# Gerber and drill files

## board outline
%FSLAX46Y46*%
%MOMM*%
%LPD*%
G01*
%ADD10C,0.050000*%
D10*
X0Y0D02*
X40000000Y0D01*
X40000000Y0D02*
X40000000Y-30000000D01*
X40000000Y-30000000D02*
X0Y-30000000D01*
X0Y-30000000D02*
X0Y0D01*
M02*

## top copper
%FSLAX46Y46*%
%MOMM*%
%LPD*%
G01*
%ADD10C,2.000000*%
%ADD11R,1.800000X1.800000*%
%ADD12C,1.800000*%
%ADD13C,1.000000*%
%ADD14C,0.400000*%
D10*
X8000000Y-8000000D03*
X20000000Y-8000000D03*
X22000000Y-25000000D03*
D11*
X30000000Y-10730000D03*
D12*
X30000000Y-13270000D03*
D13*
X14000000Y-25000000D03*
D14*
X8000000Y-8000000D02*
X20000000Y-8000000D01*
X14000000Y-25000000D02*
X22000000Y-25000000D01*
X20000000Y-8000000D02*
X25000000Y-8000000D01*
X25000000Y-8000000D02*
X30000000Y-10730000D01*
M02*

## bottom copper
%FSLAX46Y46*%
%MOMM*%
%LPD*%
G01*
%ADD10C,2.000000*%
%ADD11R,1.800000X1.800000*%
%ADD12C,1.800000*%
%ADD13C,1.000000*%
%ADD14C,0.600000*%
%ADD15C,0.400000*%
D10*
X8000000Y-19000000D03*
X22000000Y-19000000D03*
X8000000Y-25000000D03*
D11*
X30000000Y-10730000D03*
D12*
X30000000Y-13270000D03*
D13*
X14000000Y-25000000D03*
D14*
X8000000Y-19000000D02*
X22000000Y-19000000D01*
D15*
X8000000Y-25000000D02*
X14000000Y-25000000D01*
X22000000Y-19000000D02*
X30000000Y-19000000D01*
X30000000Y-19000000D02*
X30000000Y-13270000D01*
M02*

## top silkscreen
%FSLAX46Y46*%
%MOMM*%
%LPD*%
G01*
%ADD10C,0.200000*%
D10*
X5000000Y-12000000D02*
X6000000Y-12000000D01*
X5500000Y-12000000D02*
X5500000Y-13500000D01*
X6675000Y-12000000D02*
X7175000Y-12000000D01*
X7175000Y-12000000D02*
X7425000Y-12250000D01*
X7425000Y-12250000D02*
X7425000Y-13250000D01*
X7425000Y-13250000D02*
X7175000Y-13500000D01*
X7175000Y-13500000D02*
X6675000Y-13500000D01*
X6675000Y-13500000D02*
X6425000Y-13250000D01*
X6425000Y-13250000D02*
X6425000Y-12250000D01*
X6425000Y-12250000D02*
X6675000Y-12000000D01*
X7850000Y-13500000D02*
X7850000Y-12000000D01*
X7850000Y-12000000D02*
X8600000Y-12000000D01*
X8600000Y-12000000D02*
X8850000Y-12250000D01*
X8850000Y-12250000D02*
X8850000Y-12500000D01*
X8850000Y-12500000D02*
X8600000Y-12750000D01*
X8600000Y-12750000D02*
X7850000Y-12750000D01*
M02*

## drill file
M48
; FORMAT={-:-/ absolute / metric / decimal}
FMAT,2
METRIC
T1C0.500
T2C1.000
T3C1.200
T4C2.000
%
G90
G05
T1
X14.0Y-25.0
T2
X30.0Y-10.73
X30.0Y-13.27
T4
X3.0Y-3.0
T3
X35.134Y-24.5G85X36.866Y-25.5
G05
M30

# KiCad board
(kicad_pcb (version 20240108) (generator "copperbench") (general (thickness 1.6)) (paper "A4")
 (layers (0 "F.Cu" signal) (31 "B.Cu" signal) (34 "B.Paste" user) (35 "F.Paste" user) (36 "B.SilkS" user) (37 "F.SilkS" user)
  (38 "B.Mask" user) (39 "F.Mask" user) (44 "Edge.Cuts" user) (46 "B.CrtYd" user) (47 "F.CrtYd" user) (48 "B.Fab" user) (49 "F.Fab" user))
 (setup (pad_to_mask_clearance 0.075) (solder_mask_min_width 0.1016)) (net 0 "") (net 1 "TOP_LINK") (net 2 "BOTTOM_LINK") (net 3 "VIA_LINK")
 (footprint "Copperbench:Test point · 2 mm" (layer "F.Cu") (at 8 8 0)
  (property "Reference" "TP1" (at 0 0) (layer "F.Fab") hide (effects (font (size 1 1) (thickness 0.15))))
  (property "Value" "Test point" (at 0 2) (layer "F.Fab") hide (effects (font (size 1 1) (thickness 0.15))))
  (pad "1" smd circle (at 0 0 0) (size 2 2) (layers "F.Cu" "F.Paste" "F.Mask") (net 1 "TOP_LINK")))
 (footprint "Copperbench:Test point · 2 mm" (layer "F.Cu") (at 20 8 0)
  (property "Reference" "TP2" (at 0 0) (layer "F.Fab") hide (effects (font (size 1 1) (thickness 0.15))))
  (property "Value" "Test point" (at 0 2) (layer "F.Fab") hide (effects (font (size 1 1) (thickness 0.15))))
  (pad "1" smd circle (at 0 0 0) (size 2 2) (layers "F.Cu" "F.Paste" "F.Mask") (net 1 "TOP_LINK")))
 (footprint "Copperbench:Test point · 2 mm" (layer "B.Cu") (at 8 19 0)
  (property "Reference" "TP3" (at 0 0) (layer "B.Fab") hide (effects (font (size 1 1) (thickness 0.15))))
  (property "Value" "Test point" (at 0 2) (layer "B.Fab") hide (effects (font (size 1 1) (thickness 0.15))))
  (pad "1" smd circle (at 0 0 0) (size 2 2) (layers "B.Cu" "B.Paste" "B.Mask") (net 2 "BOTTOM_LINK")))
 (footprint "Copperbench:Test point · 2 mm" (layer "B.Cu") (at 22 19 0)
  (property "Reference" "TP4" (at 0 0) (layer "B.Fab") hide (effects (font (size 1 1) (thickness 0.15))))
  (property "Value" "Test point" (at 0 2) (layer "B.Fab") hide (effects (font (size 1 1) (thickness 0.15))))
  (pad "1" smd circle (at 0 0 0) (size 2 2) (layers "B.Cu" "B.Paste" "B.Mask") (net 2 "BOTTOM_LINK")))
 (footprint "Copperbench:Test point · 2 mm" (layer "B.Cu") (at 8 25 0)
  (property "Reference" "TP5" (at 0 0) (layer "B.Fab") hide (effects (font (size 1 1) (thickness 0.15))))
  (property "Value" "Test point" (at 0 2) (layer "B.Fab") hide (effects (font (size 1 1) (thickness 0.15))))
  (pad "1" smd circle (at 0 0 0) (size 2 2) (layers "B.Cu" "B.Paste" "B.Mask") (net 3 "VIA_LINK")))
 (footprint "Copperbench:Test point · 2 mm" (layer "F.Cu") (at 22 25 0)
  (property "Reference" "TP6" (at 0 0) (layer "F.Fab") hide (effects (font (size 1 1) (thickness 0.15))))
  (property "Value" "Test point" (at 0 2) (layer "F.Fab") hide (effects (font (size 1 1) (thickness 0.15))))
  (pad "1" smd circle (at 0 0 0) (size 2 2) (layers "F.Cu" "F.Paste" "F.Mask") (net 3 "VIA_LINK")))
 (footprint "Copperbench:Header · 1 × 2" (layer "F.Cu") (at 30 12 0)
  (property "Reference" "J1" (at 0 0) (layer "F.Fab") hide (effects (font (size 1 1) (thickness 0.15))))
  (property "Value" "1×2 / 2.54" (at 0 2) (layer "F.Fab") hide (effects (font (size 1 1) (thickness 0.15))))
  (pad "1" thru_hole rect (at 0 -1.27 -90) (size 1.8 1.8) (drill 1) (layers "*.Cu" "*.Mask") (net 1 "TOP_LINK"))
  (pad "2" thru_hole circle (at 0 1.27 -90) (size 1.8 1.8) (drill 1) (layers "*.Cu" "*.Mask") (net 2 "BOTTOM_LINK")))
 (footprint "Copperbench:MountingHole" (layer "F.Cu") (at 3 3)
  (pad "" np_thru_hole circle (at 0 0 0) (size 2 2) (drill 2) (layers "*.Cu" "*.Mask")))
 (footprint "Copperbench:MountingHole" (layer "F.Cu") (at 36 25)
  (pad "" np_thru_hole oval (at 0 0 -30) (size 3.2 1.2) (drill oval 3.2 1.2) (layers "*.Cu" "*.Mask")))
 (segment (start 8 8) (end 20 8) (width 0.4) (layer "F.Cu") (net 1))
 (segment (start 8 19) (end 22 19) (width 0.6) (layer "B.Cu") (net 2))
 (segment (start 8 25) (end 14 25) (width 0.4) (layer "B.Cu") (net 3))
 (segment (start 14 25) (end 22 25) (width 0.4) (layer "F.Cu") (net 3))
 (segment (start 20 8) (end 25 8) (width 0.4) (layer "F.Cu") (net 1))
 (segment (start 25 8) (end 30 10.73) (width 0.4) (layer "F.Cu") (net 1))
 (segment (start 22 19) (end 30 19) (width 0.4) (layer "B.Cu") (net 2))
 (segment (start 30 19) (end 30 13.27) (width 0.4) (layer "B.Cu") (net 2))
 (via (at 14 25) (size 1) (drill 0.5) (layers "F.Cu" "B.Cu") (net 3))
 (gr_line (start 0 0) (end 40 0) (stroke (width 0.05) (type default)) (layer "Edge.Cuts"))
 (gr_line (start 40 0) (end 40 30) (stroke (width 0.05) (type default)) (layer "Edge.Cuts"))
 (gr_line (start 40 30) (end 0 30) (stroke (width 0.05) (type default)) (layer "Edge.Cuts"))
 (gr_line (start 0 30) (end 0 0) (stroke (width 0.05) (type default)) (layer "Edge.Cuts"))
 (gr_line (start 5 12) (end 6 12) (stroke (width 0.2) (type default)) (layer "F.SilkS"))
 (gr_line (start 5.5 12) (end 5.5 13.5) (stroke (width 0.2) (type default)) (layer "F.SilkS"))
 (gr_line (start 6.675 12) (end 7.175 12) (stroke (width 0.2) (type default)) (layer "F.SilkS"))
 (gr_line (start 7.175 12) (end 7.425 12.25) (stroke (width 0.2) (type default)) (layer "F.SilkS"))
 (gr_line (start 7.425 12.25) (end 7.425 13.25) (stroke (width 0.2) (type default)) (layer "F.SilkS"))
 (gr_line (start 7.425 13.25) (end 7.175 13.5) (stroke (width 0.2) (type default)) (layer "F.SilkS"))
 (gr_line (start 7.175 13.5) (end 6.675 13.5) (stroke (width 0.2) (type default)) (layer "F.SilkS"))
 (gr_line (start 6.675 13.5) (end 6.425 13.25) (stroke (width 0.2) (type default)) (layer "F.SilkS"))
 (gr_line (start 6.425 13.25) (end 6.425 12.25) (stroke (width 0.2) (type default)) (layer "F.SilkS"))
 (gr_line (start 6.425 12.25) (end 6.675 12) (stroke (width 0.2) (type default)) (layer "F.SilkS"))
 (gr_line (start 7.85 13.5) (end 7.85 12) (stroke (width 0.2) (type default)) (layer "F.SilkS"))
 (gr_line (start 7.85 12) (end 8.6 12) (stroke (width 0.2) (type default)) (layer "F.SilkS"))
 (gr_line (start 8.6 12) (end 8.85 12.25) (stroke (width 0.2) (type default)) (layer "F.SilkS"))
 (gr_line (start 8.85 12.25) (end 8.85 12.5) (stroke (width 0.2) (type default)) (layer "F.SilkS"))
 (gr_line (start 8.85 12.5) (end 8.6 12.75) (stroke (width 0.2) (type default)) (layer "F.SilkS"))
 (gr_line (start 8.6 12.75) (end 7.85 12.75) (stroke (width 0.2) (type default)) (layer "F.SilkS")))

